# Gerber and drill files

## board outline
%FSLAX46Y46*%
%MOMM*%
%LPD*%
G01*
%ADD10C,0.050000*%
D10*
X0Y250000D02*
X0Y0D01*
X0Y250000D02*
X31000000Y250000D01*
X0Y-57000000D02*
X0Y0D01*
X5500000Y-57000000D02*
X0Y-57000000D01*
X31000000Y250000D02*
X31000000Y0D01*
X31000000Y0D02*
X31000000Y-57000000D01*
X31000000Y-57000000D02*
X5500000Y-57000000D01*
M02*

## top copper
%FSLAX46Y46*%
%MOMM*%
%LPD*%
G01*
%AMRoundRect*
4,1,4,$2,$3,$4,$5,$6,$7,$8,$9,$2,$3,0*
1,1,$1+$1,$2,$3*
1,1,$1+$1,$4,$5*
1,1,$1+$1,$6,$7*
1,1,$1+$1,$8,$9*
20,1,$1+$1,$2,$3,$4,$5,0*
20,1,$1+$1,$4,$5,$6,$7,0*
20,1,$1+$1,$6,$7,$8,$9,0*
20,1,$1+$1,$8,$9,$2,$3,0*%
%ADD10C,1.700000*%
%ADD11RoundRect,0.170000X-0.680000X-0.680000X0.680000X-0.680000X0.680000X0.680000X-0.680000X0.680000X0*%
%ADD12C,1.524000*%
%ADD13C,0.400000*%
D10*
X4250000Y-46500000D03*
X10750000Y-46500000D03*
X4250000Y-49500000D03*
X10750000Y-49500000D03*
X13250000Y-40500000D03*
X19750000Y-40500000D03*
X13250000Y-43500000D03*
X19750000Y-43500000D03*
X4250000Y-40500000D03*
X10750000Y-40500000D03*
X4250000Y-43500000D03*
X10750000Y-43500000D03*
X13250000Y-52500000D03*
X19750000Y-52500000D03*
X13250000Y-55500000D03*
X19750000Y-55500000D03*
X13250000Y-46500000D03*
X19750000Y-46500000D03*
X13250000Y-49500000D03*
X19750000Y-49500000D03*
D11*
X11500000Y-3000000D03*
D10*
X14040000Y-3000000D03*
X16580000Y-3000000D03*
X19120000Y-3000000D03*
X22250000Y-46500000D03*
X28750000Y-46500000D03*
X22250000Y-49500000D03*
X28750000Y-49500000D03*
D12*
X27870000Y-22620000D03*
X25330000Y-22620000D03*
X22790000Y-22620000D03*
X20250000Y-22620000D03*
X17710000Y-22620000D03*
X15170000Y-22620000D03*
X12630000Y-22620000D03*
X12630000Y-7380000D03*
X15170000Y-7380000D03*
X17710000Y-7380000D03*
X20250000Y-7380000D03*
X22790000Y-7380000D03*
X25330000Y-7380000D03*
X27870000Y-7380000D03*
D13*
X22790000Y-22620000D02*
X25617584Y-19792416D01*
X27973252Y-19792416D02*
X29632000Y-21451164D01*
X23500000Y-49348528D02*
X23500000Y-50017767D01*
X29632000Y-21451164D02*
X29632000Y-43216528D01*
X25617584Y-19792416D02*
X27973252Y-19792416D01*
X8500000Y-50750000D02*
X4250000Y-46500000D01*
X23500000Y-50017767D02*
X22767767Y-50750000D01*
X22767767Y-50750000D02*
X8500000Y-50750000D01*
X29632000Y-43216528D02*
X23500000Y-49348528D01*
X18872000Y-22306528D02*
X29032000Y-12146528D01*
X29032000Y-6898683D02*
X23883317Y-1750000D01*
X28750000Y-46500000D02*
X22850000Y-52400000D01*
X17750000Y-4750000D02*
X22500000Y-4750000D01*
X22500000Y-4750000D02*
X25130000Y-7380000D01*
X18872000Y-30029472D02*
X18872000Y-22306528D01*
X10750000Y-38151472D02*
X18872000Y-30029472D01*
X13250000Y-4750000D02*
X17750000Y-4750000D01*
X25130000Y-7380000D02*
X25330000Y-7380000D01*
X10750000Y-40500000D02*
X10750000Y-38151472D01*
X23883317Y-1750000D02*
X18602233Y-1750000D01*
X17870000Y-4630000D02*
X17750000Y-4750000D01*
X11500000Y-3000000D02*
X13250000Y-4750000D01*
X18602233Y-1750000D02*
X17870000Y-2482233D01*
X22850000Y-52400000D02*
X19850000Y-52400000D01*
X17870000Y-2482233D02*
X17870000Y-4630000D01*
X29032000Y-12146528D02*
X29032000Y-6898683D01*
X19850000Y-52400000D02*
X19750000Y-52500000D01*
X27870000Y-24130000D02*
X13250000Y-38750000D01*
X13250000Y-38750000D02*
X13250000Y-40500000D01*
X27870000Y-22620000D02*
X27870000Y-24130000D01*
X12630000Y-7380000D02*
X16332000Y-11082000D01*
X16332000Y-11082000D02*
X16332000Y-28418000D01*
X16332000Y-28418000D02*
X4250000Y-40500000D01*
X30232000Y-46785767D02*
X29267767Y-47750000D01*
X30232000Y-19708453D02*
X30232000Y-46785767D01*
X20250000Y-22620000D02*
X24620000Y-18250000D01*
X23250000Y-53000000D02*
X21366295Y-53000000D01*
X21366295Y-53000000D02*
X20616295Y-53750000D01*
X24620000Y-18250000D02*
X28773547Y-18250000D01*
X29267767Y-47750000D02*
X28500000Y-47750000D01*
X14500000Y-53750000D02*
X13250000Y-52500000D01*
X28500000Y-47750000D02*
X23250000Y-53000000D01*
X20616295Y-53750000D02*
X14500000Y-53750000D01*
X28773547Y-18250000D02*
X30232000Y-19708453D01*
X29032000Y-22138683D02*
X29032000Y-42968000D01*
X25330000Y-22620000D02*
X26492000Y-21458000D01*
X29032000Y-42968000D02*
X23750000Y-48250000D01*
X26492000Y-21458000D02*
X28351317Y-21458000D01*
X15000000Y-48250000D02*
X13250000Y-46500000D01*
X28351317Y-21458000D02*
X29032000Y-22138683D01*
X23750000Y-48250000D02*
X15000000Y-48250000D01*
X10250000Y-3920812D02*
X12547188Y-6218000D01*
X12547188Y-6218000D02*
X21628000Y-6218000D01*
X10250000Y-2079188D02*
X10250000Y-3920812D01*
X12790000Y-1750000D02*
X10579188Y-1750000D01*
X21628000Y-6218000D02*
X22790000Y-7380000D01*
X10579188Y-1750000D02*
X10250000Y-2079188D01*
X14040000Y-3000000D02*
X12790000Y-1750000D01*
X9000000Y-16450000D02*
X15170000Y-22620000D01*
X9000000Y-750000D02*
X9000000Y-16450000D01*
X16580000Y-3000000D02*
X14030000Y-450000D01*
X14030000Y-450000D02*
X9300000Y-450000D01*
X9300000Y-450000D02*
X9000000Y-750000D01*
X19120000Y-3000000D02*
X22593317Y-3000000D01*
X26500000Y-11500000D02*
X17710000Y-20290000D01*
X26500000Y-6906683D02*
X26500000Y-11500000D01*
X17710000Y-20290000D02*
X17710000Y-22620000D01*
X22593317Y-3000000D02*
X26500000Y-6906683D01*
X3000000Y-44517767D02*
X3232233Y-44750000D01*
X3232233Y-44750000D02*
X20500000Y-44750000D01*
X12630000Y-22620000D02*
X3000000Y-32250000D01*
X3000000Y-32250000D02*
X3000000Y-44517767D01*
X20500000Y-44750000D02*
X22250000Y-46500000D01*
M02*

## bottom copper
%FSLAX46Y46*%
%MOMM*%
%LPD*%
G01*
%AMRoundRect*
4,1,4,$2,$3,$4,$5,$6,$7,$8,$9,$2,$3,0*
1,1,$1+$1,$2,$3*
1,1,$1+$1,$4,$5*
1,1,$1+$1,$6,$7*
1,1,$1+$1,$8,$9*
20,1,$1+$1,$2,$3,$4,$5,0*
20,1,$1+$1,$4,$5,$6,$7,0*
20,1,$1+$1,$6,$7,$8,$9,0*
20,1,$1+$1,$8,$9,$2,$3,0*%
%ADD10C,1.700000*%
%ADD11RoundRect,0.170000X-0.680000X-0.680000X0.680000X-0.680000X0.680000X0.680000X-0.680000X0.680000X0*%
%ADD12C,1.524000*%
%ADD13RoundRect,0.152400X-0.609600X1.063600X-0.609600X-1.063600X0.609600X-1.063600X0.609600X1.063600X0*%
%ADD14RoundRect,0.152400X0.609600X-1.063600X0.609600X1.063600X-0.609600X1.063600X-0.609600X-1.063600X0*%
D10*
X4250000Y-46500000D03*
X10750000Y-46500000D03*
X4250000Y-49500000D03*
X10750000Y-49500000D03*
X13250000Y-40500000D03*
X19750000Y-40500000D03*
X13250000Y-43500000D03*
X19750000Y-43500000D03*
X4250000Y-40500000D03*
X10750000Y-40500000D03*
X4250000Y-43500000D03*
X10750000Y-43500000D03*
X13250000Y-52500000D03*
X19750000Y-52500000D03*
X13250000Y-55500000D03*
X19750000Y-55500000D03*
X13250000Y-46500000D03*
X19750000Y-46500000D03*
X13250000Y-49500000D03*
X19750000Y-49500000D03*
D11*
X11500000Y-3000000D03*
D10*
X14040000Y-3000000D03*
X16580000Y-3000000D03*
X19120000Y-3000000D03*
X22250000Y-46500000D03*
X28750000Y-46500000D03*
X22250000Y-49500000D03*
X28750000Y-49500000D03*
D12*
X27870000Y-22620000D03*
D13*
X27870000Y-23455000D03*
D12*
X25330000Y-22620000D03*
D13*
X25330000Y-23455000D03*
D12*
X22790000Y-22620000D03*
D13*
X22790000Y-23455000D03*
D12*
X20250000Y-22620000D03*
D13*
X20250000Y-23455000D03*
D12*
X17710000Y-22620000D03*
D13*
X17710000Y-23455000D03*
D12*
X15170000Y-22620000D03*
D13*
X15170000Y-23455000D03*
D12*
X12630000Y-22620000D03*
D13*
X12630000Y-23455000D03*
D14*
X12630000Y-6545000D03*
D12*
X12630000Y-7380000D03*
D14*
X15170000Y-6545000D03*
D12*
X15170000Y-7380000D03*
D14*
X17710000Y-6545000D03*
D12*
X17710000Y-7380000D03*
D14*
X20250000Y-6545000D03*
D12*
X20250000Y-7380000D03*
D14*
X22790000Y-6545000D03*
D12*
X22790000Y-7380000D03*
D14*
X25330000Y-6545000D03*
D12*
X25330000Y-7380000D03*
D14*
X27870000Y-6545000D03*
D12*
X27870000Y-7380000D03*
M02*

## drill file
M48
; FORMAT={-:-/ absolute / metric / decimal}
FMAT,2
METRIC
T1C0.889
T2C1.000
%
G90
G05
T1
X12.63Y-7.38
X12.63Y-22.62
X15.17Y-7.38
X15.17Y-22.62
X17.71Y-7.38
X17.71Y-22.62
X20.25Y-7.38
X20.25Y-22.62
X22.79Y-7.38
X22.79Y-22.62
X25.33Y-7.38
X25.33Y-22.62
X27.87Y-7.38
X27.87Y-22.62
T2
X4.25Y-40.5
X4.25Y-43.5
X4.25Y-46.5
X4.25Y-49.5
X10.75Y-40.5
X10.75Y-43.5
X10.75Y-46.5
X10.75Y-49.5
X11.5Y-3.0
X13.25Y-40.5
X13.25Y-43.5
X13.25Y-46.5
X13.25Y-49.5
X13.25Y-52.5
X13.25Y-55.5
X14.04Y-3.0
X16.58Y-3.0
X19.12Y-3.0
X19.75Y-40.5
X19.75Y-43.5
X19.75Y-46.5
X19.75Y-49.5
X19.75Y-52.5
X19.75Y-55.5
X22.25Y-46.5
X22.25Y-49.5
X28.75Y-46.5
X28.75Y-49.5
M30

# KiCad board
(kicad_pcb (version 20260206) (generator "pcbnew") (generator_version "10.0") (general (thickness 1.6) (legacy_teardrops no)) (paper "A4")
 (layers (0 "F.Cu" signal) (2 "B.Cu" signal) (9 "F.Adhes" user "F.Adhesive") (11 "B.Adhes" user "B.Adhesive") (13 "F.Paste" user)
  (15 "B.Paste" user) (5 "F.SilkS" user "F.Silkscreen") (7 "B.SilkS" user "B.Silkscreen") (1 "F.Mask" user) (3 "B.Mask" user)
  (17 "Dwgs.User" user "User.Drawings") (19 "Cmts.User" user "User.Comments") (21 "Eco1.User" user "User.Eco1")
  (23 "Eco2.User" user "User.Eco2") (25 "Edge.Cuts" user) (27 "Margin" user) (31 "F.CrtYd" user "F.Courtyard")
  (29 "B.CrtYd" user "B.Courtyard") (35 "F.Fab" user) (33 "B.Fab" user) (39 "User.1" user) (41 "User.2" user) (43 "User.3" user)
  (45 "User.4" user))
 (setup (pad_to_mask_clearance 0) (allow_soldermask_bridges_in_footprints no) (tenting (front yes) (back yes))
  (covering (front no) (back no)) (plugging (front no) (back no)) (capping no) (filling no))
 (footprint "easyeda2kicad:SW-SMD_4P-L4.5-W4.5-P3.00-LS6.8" (layer "F.Cu") (at 7.5 48)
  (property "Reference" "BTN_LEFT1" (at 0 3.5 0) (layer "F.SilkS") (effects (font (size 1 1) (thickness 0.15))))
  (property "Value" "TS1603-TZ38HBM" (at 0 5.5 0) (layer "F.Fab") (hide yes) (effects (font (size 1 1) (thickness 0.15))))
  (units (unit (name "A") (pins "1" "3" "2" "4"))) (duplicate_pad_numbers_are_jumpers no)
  (pad "1" thru_hole circle (at -3.25 -1.5) (size 1.7 1.7) (drill 1) (layers "*.Cu" "*.Mask") (remove_unused_layers no)
   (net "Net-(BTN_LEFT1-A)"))
  (pad "2" thru_hole circle (at 3.25 -1.5) (size 1.7 1.7) (drill 1) (layers "*.Cu" "*.Mask") (remove_unused_layers no) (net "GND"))
  (pad "3" thru_hole circle (at -3.25 1.5) (size 1.7 1.7) (drill 1) (layers "*.Cu" "*.Mask") (remove_unused_layers no)
   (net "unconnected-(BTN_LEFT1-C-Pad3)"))
  (pad "4" thru_hole circle (at 3.25 1.5) (size 1.7 1.7) (drill 1) (layers "*.Cu" "*.Mask") (remove_unused_layers no)
   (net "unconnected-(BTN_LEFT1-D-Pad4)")))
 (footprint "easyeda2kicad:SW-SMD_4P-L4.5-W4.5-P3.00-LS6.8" (layer "F.Cu") (at 16.5 42)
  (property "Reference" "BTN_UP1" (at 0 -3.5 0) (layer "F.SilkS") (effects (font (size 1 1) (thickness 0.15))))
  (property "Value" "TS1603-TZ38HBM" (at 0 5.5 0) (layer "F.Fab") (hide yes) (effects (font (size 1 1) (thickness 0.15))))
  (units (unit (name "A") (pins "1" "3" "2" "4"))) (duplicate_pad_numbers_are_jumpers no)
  (pad "1" thru_hole circle (at -3.25 -1.5) (size 1.7 1.7) (drill 1) (layers "*.Cu" "*.Mask") (remove_unused_layers no)
   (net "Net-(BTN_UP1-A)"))
  (pad "2" thru_hole circle (at 3.25 -1.5) (size 1.7 1.7) (drill 1) (layers "*.Cu" "*.Mask") (remove_unused_layers no) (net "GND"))
  (pad "3" thru_hole circle (at -3.25 1.5) (size 1.7 1.7) (drill 1) (layers "*.Cu" "*.Mask") (remove_unused_layers no)
   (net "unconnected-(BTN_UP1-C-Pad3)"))
  (pad "4" thru_hole circle (at 3.25 1.5) (size 1.7 1.7) (drill 1) (layers "*.Cu" "*.Mask") (remove_unused_layers no)
   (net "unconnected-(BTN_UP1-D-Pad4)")))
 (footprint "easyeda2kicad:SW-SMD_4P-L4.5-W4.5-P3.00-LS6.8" (layer "F.Cu") (at 7.5 42)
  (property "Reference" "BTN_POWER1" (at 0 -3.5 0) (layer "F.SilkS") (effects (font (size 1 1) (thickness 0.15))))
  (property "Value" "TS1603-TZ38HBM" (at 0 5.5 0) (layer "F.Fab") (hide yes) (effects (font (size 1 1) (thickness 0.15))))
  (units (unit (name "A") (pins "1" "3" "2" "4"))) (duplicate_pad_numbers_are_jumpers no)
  (pad "1" thru_hole circle (at -3.25 -1.5) (size 1.7 1.7) (drill 1) (layers "*.Cu" "*.Mask") (remove_unused_layers no)
   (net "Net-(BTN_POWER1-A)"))
  (pad "2" thru_hole circle (at 3.25 -1.5) (size 1.7 1.7) (drill 1) (layers "*.Cu" "*.Mask") (remove_unused_layers no) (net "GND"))
  (pad "3" thru_hole circle (at -3.25 1.5) (size 1.7 1.7) (drill 1) (layers "*.Cu" "*.Mask") (remove_unused_layers no)
   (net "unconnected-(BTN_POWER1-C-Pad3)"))
  (pad "4" thru_hole circle (at 3.25 1.5) (size 1.7 1.7) (drill 1) (layers "*.Cu" "*.Mask") (remove_unused_layers no)
   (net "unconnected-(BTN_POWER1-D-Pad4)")))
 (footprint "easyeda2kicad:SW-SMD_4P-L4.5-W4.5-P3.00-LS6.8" (layer "F.Cu") (at 16.5 54)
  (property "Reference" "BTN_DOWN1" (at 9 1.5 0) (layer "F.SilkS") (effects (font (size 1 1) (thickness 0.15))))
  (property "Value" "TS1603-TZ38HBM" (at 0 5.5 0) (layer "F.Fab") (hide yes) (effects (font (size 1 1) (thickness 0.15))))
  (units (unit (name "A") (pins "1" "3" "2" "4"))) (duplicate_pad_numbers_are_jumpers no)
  (pad "1" thru_hole circle (at -3.25 -1.5) (size 1.7 1.7) (drill 1) (layers "*.Cu" "*.Mask") (remove_unused_layers no)
   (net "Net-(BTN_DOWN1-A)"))
  (pad "2" thru_hole circle (at 3.25 -1.5) (size 1.7 1.7) (drill 1) (layers "*.Cu" "*.Mask") (remove_unused_layers no) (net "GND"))
  (pad "3" thru_hole circle (at -3.25 1.5) (size 1.7 1.7) (drill 1) (layers "*.Cu" "*.Mask") (remove_unused_layers no)
   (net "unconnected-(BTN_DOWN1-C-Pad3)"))
  (pad "4" thru_hole circle (at 3.25 1.5) (size 1.7 1.7) (drill 1) (layers "*.Cu" "*.Mask") (remove_unused_layers no)
   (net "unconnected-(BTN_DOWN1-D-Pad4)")))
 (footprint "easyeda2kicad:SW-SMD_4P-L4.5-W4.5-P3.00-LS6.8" (layer "F.Cu") (at 16.5 48)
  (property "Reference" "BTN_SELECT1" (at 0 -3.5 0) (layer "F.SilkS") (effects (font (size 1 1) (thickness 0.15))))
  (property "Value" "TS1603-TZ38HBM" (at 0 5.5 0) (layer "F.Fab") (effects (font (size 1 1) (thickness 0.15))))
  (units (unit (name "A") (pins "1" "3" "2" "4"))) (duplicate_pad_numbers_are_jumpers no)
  (pad "1" thru_hole circle (at -3.25 -1.5) (size 1.7 1.7) (drill 1) (layers "*.Cu" "*.Mask") (remove_unused_layers no)
   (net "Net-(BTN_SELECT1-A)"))
  (pad "2" thru_hole circle (at 3.25 -1.5) (size 1.7 1.7) (drill 1) (layers "*.Cu" "*.Mask") (remove_unused_layers no) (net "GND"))
  (pad "3" thru_hole circle (at -3.25 1.5) (size 1.7 1.7) (drill 1) (layers "*.Cu" "*.Mask") (remove_unused_layers no)
   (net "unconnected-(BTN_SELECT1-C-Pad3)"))
  (pad "4" thru_hole circle (at 3.25 1.5) (size 1.7 1.7) (drill 1) (layers "*.Cu" "*.Mask") (remove_unused_layers no)
   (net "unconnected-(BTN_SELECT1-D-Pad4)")))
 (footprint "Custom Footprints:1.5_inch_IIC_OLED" (layer "F.Cu") (at 11.5 3)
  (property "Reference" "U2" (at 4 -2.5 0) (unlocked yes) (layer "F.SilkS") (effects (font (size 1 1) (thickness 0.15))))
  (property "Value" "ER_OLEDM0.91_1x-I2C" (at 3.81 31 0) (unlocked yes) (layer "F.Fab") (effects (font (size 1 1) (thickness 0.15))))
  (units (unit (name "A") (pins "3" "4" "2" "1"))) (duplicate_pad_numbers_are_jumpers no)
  (pad "1" thru_hole roundrect (at 0 0) (size 1.7 1.7) (drill 1) (layers "*.Cu" "*.Mask") (remove_unused_layers no) (roundrect_rratio 0.1)
   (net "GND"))
  (pad "2" thru_hole circle (at 2.54 0) (size 1.7 1.7) (drill 1) (layers "*.Cu" "*.Mask") (remove_unused_layers no) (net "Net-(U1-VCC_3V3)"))
  (pad "3" thru_hole circle (at 5.08 0) (size 1.7 1.7) (drill 1) (layers "*.Cu" "*.Mask") (remove_unused_layers no) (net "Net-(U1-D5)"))
  (pad "4" thru_hole circle (at 7.62 0) (size 1.7 1.7) (drill 1) (layers "*.Cu" "*.Mask") (remove_unused_layers no) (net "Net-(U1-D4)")))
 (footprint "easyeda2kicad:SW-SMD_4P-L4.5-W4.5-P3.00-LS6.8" (layer "F.Cu") (at 25.5 48)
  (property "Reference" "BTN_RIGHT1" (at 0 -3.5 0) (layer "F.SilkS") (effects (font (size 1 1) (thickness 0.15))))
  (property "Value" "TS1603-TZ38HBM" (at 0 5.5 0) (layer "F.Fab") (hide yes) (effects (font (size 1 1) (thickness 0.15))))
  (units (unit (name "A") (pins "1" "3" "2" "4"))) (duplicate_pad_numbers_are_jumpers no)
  (pad "1" thru_hole circle (at -3.25 -1.5) (size 1.7 1.7) (drill 1) (layers "*.Cu" "*.Mask") (remove_unused_layers no)
   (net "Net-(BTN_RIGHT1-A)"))
  (pad "2" thru_hole circle (at 3.25 -1.5) (size 1.7 1.7) (drill 1) (layers "*.Cu" "*.Mask") (remove_unused_layers no) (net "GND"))
  (pad "3" thru_hole circle (at -3.25 1.5) (size 1.7 1.7) (drill 1) (layers "*.Cu" "*.Mask") (remove_unused_layers no)
   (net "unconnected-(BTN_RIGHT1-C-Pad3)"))
  (pad "4" thru_hole circle (at 3.25 1.5) (size 1.7 1.7) (drill 1) (layers "*.Cu" "*.Mask") (remove_unused_layers no)
   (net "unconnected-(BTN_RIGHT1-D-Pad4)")))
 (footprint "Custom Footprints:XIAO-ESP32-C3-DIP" (layer "B.Cu") (at 20.25 15)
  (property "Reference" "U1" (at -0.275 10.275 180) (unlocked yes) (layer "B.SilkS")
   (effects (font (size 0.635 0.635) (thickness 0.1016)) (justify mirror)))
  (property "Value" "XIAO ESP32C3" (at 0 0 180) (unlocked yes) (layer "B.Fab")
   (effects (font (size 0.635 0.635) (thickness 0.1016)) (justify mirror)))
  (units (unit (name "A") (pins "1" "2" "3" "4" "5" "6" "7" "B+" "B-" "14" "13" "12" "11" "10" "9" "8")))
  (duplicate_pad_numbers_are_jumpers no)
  (pad "1" thru_hole circle (at 7.62 7.62 270) (size 1.524 1.524) (drill 0.889) (layers "*.Cu" "*.Mask") (remove_unused_layers no)
   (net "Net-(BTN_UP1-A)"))
  (pad "1" smd roundrect (at 7.62 8.455 270) (size 2.432 1.524) (layers "B.Cu" "B.Mask") (roundrect_rratio 0.1) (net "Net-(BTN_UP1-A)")
   (thermal_bridge_angle 45))
  (pad "2" thru_hole circle (at 5.08 7.62 270) (size 1.524 1.524) (drill 0.889) (layers "*.Cu" "*.Mask") (remove_unused_layers no)
   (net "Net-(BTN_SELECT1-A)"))
  (pad "2" smd roundrect (at 5.08 8.455 270) (size 2.432 1.524) (layers "B.Cu" "B.Mask") (roundrect_rratio 0.1) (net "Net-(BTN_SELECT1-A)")
   (thermal_bridge_angle 45))
  (pad "3" thru_hole circle (at 2.54 7.62 270) (size 1.524 1.524) (drill 0.889) (layers "*.Cu" "*.Mask") (remove_unused_layers no)
   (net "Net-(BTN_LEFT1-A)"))
  (pad "3" smd roundrect (at 2.54 8.455 270) (size 2.432 1.524) (layers "B.Cu" "B.Mask") (roundrect_rratio 0.1) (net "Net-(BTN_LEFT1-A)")
   (thermal_bridge_angle 45))
  (pad "4" thru_hole circle (at 0 7.62 270) (size 1.524 1.524) (drill 0.889) (layers "*.Cu" "*.Mask") (remove_unused_layers no)
   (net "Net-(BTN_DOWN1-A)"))
  (pad "4" smd roundrect (at 0 8.455 270) (size 2.432 1.524) (layers "B.Cu" "B.Mask") (roundrect_rratio 0.1) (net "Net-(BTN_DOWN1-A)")
   (thermal_bridge_angle 45))
  (pad "5" thru_hole circle (at -2.54 7.62 270) (size 1.524 1.524) (drill 0.889) (layers "*.Cu" "*.Mask") (remove_unused_layers no)
   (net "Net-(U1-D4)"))
  (pad "5" smd roundrect (at -2.54 8.455 270) (size 2.432 1.524) (layers "B.Cu" "B.Mask") (roundrect_rratio 0.1) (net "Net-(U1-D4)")
   (thermal_bridge_angle 45))
  (pad "6" thru_hole circle (at -5.08 7.62 270) (size 1.524 1.524) (drill 0.889) (layers "*.Cu" "*.Mask") (remove_unused_layers no)
   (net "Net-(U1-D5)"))
  (pad "6" smd roundrect (at -5.08 8.455 270) (size 2.432 1.524) (layers "B.Cu" "B.Mask") (roundrect_rratio 0.1) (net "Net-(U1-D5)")
   (thermal_bridge_angle 45))
  (pad "7" thru_hole circle (at -7.62 7.62 270) (size 1.524 1.524) (drill 0.889) (layers "*.Cu" "*.Mask") (remove_unused_layers no)
   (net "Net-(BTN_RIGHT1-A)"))
  (pad "7" smd roundrect (at -7.62 8.455 270) (size 2.432 1.524) (layers "B.Cu" "B.Mask") (roundrect_rratio 0.1) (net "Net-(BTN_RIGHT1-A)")
   (thermal_bridge_angle 45))
  (pad "8" smd roundrect (at -7.62 -8.455 90) (size 2.432 1.524) (layers "B.Cu" "B.Mask") (roundrect_rratio 0.1) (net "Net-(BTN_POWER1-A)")
   (thermal_bridge_angle 45))
  (pad "8" thru_hole circle (at -7.62 -7.62 90) (size 1.524 1.524) (drill 0.889) (layers "*.Cu" "*.Mask") (remove_unused_layers no)
   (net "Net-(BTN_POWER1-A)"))
  (pad "9" smd roundrect (at -5.08 -8.455 90) (size 2.432 1.524) (layers "B.Cu" "B.Mask") (roundrect_rratio 0.1)
   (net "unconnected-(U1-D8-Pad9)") (thermal_bridge_angle 45))
  (pad "9" thru_hole circle (at -5.08 -7.62 90) (size 1.524 1.524) (drill 0.889) (layers "*.Cu" "*.Mask") (remove_unused_layers no)
   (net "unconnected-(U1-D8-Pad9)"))
  (pad "10" smd roundrect (at -2.54 -8.455 90) (size 2.432 1.524) (layers "B.Cu" "B.Mask") (roundrect_rratio 0.1)
   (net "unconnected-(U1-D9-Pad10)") (thermal_bridge_angle 45))
  (pad "10" thru_hole circle (at -2.54 -7.62 90) (size 1.524 1.524) (drill 0.889) (layers "*.Cu" "*.Mask") (remove_unused_layers no)
   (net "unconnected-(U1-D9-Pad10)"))
  (pad "11" smd roundrect (at 0 -8.455 90) (size 2.432 1.524) (layers "B.Cu" "B.Mask") (roundrect_rratio 0.1)
   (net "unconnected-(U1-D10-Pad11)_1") (thermal_bridge_angle 45))
  (pad "11" thru_hole circle (at 0 -7.62 90) (size 1.524 1.524) (drill 0.889) (layers "*.Cu" "*.Mask") (remove_unused_layers no)
   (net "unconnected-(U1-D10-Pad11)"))
  (pad "12" smd roundrect (at 2.54 -8.455 90) (size 2.432 1.524) (layers "B.Cu" "B.Mask") (roundrect_rratio 0.1) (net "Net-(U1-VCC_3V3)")
   (thermal_bridge_angle 45))
  (pad "12" thru_hole circle (at 2.54 -7.62 90) (size 1.524 1.524) (drill 0.889) (layers "*.Cu" "*.Mask") (remove_unused_layers no)
   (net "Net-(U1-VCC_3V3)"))
  (pad "13" smd roundrect (at 5.08 -8.455 90) (size 2.432 1.524) (layers "B.Cu" "B.Mask") (roundrect_rratio 0.1) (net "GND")
   (thermal_bridge_angle 45))
  (pad "13" thru_hole circle (at 5.08 -7.62 90) (size 1.524 1.524) (drill 0.889) (layers "*.Cu" "*.Mask") (remove_unused_layers no)
   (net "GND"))
  (pad "14" smd roundrect (at 7.62 -8.455 90) (size 2.432 1.524) (layers "B.Cu" "B.Mask") (roundrect_rratio 0.1)
   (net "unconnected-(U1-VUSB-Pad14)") (thermal_bridge_angle 45))
  (pad "14" thru_hole circle (at 7.62 -7.62 90) (size 1.524 1.524) (drill 0.889) (layers "*.Cu" "*.Mask") (remove_unused_layers no)
   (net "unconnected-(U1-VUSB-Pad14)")))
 (gr_line (start 0 -0.25) (end 0 0) (stroke (width 0.05) (type default)) (layer "Edge.Cuts"))
 (gr_line (start 0 -0.25) (end 31 -0.25) (stroke (width 0.05) (type default)) (layer "Edge.Cuts"))
 (gr_line (start 0 57) (end 0 0) (stroke (width 0.05) (type default)) (layer "Edge.Cuts"))
 (gr_line (start 5.5 57) (end 0 57) (stroke (width 0.05) (type default)) (layer "Edge.Cuts"))
 (gr_line (start 31 -0.25) (end 31 0) (stroke (width 0.05) (type default)) (layer "Edge.Cuts"))
 (gr_line (start 31 0) (end 31 57) (stroke (width 0.05) (type default)) (layer "Edge.Cuts"))
 (gr_line (start 31 57) (end 5.5 57) (stroke (width 0.05) (type default)) (layer "Edge.Cuts"))
 (segment (start 22.79 22.62) (end 25.617584 19.792416) (width 0.4) (layer "F.Cu") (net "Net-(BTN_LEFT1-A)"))
 (segment (start 27.973252 19.792416) (end 29.632 21.451164) (width 0.4) (layer "F.Cu") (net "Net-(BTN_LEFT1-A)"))
 (segment (start 23.5 49.348528) (end 23.5 50.017767) (width 0.4) (layer "F.Cu") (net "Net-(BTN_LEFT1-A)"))
 (segment (start 29.632 21.451164) (end 29.632 43.216528) (width 0.4) (layer "F.Cu") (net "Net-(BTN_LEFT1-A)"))
 (segment (start 25.617584 19.792416) (end 27.973252 19.792416) (width 0.4) (layer "F.Cu") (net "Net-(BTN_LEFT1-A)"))
 (segment (start 8.5 50.75) (end 4.25 46.5) (width 0.4) (layer "F.Cu") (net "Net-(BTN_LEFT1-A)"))
 (segment (start 23.5 50.017767) (end 22.767767 50.75) (width 0.4) (layer "F.Cu") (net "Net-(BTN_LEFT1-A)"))
 (segment (start 22.767767 50.75) (end 8.5 50.75) (width 0.4) (layer "F.Cu") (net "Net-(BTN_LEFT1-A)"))
 (segment (start 29.632 43.216528) (end 23.5 49.348528) (width 0.4) (layer "F.Cu") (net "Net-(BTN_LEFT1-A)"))
 (segment (start 18.872 22.306528) (end 29.032 12.146528) (width 0.4) (layer "F.Cu") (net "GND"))
 (segment (start 29.032 6.898683) (end 23.883317 1.75) (width 0.4) (layer "F.Cu") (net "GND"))
 (segment (start 28.75 46.5) (end 22.85 52.4) (width 0.4) (layer "F.Cu") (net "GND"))
 (segment (start 17.75 4.75) (end 22.5 4.75) (width 0.4) (layer "F.Cu") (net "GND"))
 (segment (start 22.5 4.75) (end 25.13 7.38) (width 0.4) (layer "F.Cu") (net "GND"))
 (segment (start 18.872 30.029472) (end 18.872 22.306528) (width 0.4) (layer "F.Cu") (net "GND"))
 (segment (start 10.75 38.151472) (end 18.872 30.029472) (width 0.4) (layer "F.Cu") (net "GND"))
 (segment (start 13.25 4.75) (end 17.75 4.75) (width 0.4) (layer "F.Cu") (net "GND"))
 (segment (start 25.13 7.38) (end 25.33 7.38) (width 0.4) (layer "F.Cu") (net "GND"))
 (segment (start 10.75 40.5) (end 10.75 38.151472) (width 0.4) (layer "F.Cu") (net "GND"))
 (segment (start 23.883317 1.75) (end 18.602233 1.75) (width 0.4) (layer "F.Cu") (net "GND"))
 (segment (start 17.87 4.63) (end 17.75 4.75) (width 0.4) (layer "F.Cu") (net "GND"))
 (segment (start 11.5 3) (end 13.25 4.75) (width 0.4) (layer "F.Cu") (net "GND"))
 (segment (start 18.602233 1.75) (end 17.87 2.482233) (width 0.4) (layer "F.Cu") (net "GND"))
 (segment (start 22.85 52.4) (end 19.85 52.4) (width 0.4) (layer "F.Cu") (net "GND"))
 (segment (start 17.87 2.482233) (end 17.87 4.63) (width 0.4) (layer "F.Cu") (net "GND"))
 (segment (start 29.032 12.146528) (end 29.032 6.898683) (width 0.4) (layer "F.Cu") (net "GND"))
 (segment (start 19.85 52.4) (end 19.75 52.5) (width 0.4) (layer "F.Cu") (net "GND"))
 (segment (start 27.87 24.13) (end 13.25 38.75) (width 0.4) (layer "F.Cu") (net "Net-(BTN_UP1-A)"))
 (segment (start 13.25 38.75) (end 13.25 40.5) (width 0.4) (layer "F.Cu") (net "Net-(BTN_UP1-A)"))
 (segment (start 27.87 22.62) (end 27.87 24.13) (width 0.4) (layer "F.Cu") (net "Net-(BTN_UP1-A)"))
 (segment (start 12.63 7.38) (end 16.332 11.082) (width 0.4) (layer "F.Cu") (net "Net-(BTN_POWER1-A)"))
 (segment (start 16.332 11.082) (end 16.332 28.418) (width 0.4) (layer "F.Cu") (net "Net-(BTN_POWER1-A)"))
 (segment (start 16.332 28.418) (end 4.25 40.5) (width 0.4) (layer "F.Cu") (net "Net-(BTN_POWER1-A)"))
 (segment (start 30.232 46.785767) (end 29.267767 47.75) (width 0.4) (layer "F.Cu") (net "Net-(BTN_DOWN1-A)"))
 (segment (start 30.232 19.708453) (end 30.232 46.785767) (width 0.4) (layer "F.Cu") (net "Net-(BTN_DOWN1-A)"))
 (segment (start 20.25 22.62) (end 24.62 18.25) (width 0.4) (layer "F.Cu") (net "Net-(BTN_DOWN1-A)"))
 (segment (start 23.25 53) (end 21.366295 53) (width 0.4) (layer "F.Cu") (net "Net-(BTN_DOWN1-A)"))
 (segment (start 21.366295 53) (end 20.616295 53.75) (width 0.4) (layer "F.Cu") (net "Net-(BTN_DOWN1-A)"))
 (segment (start 24.62 18.25) (end 28.773547 18.25) (width 0.4) (layer "F.Cu") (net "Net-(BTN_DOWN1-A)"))
 (segment (start 29.267767 47.75) (end 28.5 47.75) (width 0.4) (layer "F.Cu") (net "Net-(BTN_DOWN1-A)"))
 (segment (start 14.5 53.75) (end 13.25 52.5) (width 0.4) (layer "F.Cu") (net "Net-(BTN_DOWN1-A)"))
 (segment (start 28.5 47.75) (end 23.25 53) (width 0.4) (layer "F.Cu") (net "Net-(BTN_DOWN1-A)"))
 (segment (start 20.616295 53.75) (end 14.5 53.75) (width 0.4) (layer "F.Cu") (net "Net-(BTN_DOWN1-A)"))
 (segment (start 28.773547 18.25) (end 30.232 19.708453) (width 0.4) (layer "F.Cu") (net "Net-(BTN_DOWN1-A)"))
 (segment (start 29.032 22.138683) (end 29.032 42.968) (width 0.4) (layer "F.Cu") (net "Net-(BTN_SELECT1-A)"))
 (segment (start 25.33 22.62) (end 26.492 21.458) (width 0.4) (layer "F.Cu") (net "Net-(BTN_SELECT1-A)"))
 (segment (start 29.032 42.968) (end 23.75 48.25) (width 0.4) (layer "F.Cu") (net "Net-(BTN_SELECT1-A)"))
 (segment (start 26.492 21.458) (end 28.351317 21.458) (width 0.4) (layer "F.Cu") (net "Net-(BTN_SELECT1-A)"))
 (segment (start 15 48.25) (end 13.25 46.5) (width 0.4) (layer "F.Cu") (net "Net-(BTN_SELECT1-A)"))
 (segment (start 28.351317 21.458) (end 29.032 22.138683) (width 0.4) (layer "F.Cu") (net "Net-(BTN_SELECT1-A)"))
 (segment (start 23.75 48.25) (end 15 48.25) (width 0.4) (layer "F.Cu") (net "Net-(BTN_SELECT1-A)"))
 (segment (start 10.25 3.920812) (end 12.547188 6.218) (width 0.4) (layer "F.Cu") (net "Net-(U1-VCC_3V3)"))
 (segment (start 12.547188 6.218) (end 21.628 6.218) (width 0.4) (layer "F.Cu") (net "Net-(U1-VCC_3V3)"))
 (segment (start 10.25 2.079188) (end 10.25 3.920812) (width 0.4) (layer "F.Cu") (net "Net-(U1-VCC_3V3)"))
 (segment (start 12.79 1.75) (end 10.579188 1.75) (width 0.4) (layer "F.Cu") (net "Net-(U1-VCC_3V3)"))
 (segment (start 21.628 6.218) (end 22.79 7.38) (width 0.4) (layer "F.Cu") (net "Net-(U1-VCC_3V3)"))
 (segment (start 10.579188 1.75) (end 10.25 2.079188) (width 0.4) (layer "F.Cu") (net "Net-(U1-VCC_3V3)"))
 (segment (start 14.04 3) (end 12.79 1.75) (width 0.4) (layer "F.Cu") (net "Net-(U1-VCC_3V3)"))
 (segment (start 9 16.45) (end 15.17 22.62) (width 0.4) (layer "F.Cu") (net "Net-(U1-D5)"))
 (segment (start 9 0.75) (end 9 16.45) (width 0.4) (layer "F.Cu") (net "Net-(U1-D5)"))
 (segment (start 16.58 3) (end 14.03 0.45) (width 0.4) (layer "F.Cu") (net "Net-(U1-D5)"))
 (segment (start 14.03 0.45) (end 9.3 0.45) (width 0.4) (layer "F.Cu") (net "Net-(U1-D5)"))
 (segment (start 9.3 0.45) (end 9 0.75) (width 0.4) (layer "F.Cu") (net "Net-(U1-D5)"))
 (segment (start 19.12 3) (end 22.593317 3) (width 0.4) (layer "F.Cu") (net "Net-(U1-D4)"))
 (segment (start 26.5 11.5) (end 17.71 20.29) (width 0.4) (layer "F.Cu") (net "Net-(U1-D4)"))
 (segment (start 26.5 6.906683) (end 26.5 11.5) (width 0.4) (layer "F.Cu") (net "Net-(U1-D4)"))
 (segment (start 17.71 20.29) (end 17.71 22.62) (width 0.4) (layer "F.Cu") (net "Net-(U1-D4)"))
 (segment (start 22.593317 3) (end 26.5 6.906683) (width 0.4) (layer "F.Cu") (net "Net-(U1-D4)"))
 (segment (start 3 44.517767) (end 3.232233 44.75) (width 0.4) (layer "F.Cu") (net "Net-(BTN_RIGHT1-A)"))
 (segment (start 3.232233 44.75) (end 20.5 44.75) (width 0.4) (layer "F.Cu") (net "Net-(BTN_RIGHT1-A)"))
 (segment (start 12.63 22.62) (end 3 32.25) (width 0.4) (layer "F.Cu") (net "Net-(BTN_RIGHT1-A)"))
 (segment (start 3 32.25) (end 3 44.517767) (width 0.4) (layer "F.Cu") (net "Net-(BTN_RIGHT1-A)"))
 (segment (start 20.5 44.75) (end 22.25 46.5) (width 0.4) (layer "F.Cu") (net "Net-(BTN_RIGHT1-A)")))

